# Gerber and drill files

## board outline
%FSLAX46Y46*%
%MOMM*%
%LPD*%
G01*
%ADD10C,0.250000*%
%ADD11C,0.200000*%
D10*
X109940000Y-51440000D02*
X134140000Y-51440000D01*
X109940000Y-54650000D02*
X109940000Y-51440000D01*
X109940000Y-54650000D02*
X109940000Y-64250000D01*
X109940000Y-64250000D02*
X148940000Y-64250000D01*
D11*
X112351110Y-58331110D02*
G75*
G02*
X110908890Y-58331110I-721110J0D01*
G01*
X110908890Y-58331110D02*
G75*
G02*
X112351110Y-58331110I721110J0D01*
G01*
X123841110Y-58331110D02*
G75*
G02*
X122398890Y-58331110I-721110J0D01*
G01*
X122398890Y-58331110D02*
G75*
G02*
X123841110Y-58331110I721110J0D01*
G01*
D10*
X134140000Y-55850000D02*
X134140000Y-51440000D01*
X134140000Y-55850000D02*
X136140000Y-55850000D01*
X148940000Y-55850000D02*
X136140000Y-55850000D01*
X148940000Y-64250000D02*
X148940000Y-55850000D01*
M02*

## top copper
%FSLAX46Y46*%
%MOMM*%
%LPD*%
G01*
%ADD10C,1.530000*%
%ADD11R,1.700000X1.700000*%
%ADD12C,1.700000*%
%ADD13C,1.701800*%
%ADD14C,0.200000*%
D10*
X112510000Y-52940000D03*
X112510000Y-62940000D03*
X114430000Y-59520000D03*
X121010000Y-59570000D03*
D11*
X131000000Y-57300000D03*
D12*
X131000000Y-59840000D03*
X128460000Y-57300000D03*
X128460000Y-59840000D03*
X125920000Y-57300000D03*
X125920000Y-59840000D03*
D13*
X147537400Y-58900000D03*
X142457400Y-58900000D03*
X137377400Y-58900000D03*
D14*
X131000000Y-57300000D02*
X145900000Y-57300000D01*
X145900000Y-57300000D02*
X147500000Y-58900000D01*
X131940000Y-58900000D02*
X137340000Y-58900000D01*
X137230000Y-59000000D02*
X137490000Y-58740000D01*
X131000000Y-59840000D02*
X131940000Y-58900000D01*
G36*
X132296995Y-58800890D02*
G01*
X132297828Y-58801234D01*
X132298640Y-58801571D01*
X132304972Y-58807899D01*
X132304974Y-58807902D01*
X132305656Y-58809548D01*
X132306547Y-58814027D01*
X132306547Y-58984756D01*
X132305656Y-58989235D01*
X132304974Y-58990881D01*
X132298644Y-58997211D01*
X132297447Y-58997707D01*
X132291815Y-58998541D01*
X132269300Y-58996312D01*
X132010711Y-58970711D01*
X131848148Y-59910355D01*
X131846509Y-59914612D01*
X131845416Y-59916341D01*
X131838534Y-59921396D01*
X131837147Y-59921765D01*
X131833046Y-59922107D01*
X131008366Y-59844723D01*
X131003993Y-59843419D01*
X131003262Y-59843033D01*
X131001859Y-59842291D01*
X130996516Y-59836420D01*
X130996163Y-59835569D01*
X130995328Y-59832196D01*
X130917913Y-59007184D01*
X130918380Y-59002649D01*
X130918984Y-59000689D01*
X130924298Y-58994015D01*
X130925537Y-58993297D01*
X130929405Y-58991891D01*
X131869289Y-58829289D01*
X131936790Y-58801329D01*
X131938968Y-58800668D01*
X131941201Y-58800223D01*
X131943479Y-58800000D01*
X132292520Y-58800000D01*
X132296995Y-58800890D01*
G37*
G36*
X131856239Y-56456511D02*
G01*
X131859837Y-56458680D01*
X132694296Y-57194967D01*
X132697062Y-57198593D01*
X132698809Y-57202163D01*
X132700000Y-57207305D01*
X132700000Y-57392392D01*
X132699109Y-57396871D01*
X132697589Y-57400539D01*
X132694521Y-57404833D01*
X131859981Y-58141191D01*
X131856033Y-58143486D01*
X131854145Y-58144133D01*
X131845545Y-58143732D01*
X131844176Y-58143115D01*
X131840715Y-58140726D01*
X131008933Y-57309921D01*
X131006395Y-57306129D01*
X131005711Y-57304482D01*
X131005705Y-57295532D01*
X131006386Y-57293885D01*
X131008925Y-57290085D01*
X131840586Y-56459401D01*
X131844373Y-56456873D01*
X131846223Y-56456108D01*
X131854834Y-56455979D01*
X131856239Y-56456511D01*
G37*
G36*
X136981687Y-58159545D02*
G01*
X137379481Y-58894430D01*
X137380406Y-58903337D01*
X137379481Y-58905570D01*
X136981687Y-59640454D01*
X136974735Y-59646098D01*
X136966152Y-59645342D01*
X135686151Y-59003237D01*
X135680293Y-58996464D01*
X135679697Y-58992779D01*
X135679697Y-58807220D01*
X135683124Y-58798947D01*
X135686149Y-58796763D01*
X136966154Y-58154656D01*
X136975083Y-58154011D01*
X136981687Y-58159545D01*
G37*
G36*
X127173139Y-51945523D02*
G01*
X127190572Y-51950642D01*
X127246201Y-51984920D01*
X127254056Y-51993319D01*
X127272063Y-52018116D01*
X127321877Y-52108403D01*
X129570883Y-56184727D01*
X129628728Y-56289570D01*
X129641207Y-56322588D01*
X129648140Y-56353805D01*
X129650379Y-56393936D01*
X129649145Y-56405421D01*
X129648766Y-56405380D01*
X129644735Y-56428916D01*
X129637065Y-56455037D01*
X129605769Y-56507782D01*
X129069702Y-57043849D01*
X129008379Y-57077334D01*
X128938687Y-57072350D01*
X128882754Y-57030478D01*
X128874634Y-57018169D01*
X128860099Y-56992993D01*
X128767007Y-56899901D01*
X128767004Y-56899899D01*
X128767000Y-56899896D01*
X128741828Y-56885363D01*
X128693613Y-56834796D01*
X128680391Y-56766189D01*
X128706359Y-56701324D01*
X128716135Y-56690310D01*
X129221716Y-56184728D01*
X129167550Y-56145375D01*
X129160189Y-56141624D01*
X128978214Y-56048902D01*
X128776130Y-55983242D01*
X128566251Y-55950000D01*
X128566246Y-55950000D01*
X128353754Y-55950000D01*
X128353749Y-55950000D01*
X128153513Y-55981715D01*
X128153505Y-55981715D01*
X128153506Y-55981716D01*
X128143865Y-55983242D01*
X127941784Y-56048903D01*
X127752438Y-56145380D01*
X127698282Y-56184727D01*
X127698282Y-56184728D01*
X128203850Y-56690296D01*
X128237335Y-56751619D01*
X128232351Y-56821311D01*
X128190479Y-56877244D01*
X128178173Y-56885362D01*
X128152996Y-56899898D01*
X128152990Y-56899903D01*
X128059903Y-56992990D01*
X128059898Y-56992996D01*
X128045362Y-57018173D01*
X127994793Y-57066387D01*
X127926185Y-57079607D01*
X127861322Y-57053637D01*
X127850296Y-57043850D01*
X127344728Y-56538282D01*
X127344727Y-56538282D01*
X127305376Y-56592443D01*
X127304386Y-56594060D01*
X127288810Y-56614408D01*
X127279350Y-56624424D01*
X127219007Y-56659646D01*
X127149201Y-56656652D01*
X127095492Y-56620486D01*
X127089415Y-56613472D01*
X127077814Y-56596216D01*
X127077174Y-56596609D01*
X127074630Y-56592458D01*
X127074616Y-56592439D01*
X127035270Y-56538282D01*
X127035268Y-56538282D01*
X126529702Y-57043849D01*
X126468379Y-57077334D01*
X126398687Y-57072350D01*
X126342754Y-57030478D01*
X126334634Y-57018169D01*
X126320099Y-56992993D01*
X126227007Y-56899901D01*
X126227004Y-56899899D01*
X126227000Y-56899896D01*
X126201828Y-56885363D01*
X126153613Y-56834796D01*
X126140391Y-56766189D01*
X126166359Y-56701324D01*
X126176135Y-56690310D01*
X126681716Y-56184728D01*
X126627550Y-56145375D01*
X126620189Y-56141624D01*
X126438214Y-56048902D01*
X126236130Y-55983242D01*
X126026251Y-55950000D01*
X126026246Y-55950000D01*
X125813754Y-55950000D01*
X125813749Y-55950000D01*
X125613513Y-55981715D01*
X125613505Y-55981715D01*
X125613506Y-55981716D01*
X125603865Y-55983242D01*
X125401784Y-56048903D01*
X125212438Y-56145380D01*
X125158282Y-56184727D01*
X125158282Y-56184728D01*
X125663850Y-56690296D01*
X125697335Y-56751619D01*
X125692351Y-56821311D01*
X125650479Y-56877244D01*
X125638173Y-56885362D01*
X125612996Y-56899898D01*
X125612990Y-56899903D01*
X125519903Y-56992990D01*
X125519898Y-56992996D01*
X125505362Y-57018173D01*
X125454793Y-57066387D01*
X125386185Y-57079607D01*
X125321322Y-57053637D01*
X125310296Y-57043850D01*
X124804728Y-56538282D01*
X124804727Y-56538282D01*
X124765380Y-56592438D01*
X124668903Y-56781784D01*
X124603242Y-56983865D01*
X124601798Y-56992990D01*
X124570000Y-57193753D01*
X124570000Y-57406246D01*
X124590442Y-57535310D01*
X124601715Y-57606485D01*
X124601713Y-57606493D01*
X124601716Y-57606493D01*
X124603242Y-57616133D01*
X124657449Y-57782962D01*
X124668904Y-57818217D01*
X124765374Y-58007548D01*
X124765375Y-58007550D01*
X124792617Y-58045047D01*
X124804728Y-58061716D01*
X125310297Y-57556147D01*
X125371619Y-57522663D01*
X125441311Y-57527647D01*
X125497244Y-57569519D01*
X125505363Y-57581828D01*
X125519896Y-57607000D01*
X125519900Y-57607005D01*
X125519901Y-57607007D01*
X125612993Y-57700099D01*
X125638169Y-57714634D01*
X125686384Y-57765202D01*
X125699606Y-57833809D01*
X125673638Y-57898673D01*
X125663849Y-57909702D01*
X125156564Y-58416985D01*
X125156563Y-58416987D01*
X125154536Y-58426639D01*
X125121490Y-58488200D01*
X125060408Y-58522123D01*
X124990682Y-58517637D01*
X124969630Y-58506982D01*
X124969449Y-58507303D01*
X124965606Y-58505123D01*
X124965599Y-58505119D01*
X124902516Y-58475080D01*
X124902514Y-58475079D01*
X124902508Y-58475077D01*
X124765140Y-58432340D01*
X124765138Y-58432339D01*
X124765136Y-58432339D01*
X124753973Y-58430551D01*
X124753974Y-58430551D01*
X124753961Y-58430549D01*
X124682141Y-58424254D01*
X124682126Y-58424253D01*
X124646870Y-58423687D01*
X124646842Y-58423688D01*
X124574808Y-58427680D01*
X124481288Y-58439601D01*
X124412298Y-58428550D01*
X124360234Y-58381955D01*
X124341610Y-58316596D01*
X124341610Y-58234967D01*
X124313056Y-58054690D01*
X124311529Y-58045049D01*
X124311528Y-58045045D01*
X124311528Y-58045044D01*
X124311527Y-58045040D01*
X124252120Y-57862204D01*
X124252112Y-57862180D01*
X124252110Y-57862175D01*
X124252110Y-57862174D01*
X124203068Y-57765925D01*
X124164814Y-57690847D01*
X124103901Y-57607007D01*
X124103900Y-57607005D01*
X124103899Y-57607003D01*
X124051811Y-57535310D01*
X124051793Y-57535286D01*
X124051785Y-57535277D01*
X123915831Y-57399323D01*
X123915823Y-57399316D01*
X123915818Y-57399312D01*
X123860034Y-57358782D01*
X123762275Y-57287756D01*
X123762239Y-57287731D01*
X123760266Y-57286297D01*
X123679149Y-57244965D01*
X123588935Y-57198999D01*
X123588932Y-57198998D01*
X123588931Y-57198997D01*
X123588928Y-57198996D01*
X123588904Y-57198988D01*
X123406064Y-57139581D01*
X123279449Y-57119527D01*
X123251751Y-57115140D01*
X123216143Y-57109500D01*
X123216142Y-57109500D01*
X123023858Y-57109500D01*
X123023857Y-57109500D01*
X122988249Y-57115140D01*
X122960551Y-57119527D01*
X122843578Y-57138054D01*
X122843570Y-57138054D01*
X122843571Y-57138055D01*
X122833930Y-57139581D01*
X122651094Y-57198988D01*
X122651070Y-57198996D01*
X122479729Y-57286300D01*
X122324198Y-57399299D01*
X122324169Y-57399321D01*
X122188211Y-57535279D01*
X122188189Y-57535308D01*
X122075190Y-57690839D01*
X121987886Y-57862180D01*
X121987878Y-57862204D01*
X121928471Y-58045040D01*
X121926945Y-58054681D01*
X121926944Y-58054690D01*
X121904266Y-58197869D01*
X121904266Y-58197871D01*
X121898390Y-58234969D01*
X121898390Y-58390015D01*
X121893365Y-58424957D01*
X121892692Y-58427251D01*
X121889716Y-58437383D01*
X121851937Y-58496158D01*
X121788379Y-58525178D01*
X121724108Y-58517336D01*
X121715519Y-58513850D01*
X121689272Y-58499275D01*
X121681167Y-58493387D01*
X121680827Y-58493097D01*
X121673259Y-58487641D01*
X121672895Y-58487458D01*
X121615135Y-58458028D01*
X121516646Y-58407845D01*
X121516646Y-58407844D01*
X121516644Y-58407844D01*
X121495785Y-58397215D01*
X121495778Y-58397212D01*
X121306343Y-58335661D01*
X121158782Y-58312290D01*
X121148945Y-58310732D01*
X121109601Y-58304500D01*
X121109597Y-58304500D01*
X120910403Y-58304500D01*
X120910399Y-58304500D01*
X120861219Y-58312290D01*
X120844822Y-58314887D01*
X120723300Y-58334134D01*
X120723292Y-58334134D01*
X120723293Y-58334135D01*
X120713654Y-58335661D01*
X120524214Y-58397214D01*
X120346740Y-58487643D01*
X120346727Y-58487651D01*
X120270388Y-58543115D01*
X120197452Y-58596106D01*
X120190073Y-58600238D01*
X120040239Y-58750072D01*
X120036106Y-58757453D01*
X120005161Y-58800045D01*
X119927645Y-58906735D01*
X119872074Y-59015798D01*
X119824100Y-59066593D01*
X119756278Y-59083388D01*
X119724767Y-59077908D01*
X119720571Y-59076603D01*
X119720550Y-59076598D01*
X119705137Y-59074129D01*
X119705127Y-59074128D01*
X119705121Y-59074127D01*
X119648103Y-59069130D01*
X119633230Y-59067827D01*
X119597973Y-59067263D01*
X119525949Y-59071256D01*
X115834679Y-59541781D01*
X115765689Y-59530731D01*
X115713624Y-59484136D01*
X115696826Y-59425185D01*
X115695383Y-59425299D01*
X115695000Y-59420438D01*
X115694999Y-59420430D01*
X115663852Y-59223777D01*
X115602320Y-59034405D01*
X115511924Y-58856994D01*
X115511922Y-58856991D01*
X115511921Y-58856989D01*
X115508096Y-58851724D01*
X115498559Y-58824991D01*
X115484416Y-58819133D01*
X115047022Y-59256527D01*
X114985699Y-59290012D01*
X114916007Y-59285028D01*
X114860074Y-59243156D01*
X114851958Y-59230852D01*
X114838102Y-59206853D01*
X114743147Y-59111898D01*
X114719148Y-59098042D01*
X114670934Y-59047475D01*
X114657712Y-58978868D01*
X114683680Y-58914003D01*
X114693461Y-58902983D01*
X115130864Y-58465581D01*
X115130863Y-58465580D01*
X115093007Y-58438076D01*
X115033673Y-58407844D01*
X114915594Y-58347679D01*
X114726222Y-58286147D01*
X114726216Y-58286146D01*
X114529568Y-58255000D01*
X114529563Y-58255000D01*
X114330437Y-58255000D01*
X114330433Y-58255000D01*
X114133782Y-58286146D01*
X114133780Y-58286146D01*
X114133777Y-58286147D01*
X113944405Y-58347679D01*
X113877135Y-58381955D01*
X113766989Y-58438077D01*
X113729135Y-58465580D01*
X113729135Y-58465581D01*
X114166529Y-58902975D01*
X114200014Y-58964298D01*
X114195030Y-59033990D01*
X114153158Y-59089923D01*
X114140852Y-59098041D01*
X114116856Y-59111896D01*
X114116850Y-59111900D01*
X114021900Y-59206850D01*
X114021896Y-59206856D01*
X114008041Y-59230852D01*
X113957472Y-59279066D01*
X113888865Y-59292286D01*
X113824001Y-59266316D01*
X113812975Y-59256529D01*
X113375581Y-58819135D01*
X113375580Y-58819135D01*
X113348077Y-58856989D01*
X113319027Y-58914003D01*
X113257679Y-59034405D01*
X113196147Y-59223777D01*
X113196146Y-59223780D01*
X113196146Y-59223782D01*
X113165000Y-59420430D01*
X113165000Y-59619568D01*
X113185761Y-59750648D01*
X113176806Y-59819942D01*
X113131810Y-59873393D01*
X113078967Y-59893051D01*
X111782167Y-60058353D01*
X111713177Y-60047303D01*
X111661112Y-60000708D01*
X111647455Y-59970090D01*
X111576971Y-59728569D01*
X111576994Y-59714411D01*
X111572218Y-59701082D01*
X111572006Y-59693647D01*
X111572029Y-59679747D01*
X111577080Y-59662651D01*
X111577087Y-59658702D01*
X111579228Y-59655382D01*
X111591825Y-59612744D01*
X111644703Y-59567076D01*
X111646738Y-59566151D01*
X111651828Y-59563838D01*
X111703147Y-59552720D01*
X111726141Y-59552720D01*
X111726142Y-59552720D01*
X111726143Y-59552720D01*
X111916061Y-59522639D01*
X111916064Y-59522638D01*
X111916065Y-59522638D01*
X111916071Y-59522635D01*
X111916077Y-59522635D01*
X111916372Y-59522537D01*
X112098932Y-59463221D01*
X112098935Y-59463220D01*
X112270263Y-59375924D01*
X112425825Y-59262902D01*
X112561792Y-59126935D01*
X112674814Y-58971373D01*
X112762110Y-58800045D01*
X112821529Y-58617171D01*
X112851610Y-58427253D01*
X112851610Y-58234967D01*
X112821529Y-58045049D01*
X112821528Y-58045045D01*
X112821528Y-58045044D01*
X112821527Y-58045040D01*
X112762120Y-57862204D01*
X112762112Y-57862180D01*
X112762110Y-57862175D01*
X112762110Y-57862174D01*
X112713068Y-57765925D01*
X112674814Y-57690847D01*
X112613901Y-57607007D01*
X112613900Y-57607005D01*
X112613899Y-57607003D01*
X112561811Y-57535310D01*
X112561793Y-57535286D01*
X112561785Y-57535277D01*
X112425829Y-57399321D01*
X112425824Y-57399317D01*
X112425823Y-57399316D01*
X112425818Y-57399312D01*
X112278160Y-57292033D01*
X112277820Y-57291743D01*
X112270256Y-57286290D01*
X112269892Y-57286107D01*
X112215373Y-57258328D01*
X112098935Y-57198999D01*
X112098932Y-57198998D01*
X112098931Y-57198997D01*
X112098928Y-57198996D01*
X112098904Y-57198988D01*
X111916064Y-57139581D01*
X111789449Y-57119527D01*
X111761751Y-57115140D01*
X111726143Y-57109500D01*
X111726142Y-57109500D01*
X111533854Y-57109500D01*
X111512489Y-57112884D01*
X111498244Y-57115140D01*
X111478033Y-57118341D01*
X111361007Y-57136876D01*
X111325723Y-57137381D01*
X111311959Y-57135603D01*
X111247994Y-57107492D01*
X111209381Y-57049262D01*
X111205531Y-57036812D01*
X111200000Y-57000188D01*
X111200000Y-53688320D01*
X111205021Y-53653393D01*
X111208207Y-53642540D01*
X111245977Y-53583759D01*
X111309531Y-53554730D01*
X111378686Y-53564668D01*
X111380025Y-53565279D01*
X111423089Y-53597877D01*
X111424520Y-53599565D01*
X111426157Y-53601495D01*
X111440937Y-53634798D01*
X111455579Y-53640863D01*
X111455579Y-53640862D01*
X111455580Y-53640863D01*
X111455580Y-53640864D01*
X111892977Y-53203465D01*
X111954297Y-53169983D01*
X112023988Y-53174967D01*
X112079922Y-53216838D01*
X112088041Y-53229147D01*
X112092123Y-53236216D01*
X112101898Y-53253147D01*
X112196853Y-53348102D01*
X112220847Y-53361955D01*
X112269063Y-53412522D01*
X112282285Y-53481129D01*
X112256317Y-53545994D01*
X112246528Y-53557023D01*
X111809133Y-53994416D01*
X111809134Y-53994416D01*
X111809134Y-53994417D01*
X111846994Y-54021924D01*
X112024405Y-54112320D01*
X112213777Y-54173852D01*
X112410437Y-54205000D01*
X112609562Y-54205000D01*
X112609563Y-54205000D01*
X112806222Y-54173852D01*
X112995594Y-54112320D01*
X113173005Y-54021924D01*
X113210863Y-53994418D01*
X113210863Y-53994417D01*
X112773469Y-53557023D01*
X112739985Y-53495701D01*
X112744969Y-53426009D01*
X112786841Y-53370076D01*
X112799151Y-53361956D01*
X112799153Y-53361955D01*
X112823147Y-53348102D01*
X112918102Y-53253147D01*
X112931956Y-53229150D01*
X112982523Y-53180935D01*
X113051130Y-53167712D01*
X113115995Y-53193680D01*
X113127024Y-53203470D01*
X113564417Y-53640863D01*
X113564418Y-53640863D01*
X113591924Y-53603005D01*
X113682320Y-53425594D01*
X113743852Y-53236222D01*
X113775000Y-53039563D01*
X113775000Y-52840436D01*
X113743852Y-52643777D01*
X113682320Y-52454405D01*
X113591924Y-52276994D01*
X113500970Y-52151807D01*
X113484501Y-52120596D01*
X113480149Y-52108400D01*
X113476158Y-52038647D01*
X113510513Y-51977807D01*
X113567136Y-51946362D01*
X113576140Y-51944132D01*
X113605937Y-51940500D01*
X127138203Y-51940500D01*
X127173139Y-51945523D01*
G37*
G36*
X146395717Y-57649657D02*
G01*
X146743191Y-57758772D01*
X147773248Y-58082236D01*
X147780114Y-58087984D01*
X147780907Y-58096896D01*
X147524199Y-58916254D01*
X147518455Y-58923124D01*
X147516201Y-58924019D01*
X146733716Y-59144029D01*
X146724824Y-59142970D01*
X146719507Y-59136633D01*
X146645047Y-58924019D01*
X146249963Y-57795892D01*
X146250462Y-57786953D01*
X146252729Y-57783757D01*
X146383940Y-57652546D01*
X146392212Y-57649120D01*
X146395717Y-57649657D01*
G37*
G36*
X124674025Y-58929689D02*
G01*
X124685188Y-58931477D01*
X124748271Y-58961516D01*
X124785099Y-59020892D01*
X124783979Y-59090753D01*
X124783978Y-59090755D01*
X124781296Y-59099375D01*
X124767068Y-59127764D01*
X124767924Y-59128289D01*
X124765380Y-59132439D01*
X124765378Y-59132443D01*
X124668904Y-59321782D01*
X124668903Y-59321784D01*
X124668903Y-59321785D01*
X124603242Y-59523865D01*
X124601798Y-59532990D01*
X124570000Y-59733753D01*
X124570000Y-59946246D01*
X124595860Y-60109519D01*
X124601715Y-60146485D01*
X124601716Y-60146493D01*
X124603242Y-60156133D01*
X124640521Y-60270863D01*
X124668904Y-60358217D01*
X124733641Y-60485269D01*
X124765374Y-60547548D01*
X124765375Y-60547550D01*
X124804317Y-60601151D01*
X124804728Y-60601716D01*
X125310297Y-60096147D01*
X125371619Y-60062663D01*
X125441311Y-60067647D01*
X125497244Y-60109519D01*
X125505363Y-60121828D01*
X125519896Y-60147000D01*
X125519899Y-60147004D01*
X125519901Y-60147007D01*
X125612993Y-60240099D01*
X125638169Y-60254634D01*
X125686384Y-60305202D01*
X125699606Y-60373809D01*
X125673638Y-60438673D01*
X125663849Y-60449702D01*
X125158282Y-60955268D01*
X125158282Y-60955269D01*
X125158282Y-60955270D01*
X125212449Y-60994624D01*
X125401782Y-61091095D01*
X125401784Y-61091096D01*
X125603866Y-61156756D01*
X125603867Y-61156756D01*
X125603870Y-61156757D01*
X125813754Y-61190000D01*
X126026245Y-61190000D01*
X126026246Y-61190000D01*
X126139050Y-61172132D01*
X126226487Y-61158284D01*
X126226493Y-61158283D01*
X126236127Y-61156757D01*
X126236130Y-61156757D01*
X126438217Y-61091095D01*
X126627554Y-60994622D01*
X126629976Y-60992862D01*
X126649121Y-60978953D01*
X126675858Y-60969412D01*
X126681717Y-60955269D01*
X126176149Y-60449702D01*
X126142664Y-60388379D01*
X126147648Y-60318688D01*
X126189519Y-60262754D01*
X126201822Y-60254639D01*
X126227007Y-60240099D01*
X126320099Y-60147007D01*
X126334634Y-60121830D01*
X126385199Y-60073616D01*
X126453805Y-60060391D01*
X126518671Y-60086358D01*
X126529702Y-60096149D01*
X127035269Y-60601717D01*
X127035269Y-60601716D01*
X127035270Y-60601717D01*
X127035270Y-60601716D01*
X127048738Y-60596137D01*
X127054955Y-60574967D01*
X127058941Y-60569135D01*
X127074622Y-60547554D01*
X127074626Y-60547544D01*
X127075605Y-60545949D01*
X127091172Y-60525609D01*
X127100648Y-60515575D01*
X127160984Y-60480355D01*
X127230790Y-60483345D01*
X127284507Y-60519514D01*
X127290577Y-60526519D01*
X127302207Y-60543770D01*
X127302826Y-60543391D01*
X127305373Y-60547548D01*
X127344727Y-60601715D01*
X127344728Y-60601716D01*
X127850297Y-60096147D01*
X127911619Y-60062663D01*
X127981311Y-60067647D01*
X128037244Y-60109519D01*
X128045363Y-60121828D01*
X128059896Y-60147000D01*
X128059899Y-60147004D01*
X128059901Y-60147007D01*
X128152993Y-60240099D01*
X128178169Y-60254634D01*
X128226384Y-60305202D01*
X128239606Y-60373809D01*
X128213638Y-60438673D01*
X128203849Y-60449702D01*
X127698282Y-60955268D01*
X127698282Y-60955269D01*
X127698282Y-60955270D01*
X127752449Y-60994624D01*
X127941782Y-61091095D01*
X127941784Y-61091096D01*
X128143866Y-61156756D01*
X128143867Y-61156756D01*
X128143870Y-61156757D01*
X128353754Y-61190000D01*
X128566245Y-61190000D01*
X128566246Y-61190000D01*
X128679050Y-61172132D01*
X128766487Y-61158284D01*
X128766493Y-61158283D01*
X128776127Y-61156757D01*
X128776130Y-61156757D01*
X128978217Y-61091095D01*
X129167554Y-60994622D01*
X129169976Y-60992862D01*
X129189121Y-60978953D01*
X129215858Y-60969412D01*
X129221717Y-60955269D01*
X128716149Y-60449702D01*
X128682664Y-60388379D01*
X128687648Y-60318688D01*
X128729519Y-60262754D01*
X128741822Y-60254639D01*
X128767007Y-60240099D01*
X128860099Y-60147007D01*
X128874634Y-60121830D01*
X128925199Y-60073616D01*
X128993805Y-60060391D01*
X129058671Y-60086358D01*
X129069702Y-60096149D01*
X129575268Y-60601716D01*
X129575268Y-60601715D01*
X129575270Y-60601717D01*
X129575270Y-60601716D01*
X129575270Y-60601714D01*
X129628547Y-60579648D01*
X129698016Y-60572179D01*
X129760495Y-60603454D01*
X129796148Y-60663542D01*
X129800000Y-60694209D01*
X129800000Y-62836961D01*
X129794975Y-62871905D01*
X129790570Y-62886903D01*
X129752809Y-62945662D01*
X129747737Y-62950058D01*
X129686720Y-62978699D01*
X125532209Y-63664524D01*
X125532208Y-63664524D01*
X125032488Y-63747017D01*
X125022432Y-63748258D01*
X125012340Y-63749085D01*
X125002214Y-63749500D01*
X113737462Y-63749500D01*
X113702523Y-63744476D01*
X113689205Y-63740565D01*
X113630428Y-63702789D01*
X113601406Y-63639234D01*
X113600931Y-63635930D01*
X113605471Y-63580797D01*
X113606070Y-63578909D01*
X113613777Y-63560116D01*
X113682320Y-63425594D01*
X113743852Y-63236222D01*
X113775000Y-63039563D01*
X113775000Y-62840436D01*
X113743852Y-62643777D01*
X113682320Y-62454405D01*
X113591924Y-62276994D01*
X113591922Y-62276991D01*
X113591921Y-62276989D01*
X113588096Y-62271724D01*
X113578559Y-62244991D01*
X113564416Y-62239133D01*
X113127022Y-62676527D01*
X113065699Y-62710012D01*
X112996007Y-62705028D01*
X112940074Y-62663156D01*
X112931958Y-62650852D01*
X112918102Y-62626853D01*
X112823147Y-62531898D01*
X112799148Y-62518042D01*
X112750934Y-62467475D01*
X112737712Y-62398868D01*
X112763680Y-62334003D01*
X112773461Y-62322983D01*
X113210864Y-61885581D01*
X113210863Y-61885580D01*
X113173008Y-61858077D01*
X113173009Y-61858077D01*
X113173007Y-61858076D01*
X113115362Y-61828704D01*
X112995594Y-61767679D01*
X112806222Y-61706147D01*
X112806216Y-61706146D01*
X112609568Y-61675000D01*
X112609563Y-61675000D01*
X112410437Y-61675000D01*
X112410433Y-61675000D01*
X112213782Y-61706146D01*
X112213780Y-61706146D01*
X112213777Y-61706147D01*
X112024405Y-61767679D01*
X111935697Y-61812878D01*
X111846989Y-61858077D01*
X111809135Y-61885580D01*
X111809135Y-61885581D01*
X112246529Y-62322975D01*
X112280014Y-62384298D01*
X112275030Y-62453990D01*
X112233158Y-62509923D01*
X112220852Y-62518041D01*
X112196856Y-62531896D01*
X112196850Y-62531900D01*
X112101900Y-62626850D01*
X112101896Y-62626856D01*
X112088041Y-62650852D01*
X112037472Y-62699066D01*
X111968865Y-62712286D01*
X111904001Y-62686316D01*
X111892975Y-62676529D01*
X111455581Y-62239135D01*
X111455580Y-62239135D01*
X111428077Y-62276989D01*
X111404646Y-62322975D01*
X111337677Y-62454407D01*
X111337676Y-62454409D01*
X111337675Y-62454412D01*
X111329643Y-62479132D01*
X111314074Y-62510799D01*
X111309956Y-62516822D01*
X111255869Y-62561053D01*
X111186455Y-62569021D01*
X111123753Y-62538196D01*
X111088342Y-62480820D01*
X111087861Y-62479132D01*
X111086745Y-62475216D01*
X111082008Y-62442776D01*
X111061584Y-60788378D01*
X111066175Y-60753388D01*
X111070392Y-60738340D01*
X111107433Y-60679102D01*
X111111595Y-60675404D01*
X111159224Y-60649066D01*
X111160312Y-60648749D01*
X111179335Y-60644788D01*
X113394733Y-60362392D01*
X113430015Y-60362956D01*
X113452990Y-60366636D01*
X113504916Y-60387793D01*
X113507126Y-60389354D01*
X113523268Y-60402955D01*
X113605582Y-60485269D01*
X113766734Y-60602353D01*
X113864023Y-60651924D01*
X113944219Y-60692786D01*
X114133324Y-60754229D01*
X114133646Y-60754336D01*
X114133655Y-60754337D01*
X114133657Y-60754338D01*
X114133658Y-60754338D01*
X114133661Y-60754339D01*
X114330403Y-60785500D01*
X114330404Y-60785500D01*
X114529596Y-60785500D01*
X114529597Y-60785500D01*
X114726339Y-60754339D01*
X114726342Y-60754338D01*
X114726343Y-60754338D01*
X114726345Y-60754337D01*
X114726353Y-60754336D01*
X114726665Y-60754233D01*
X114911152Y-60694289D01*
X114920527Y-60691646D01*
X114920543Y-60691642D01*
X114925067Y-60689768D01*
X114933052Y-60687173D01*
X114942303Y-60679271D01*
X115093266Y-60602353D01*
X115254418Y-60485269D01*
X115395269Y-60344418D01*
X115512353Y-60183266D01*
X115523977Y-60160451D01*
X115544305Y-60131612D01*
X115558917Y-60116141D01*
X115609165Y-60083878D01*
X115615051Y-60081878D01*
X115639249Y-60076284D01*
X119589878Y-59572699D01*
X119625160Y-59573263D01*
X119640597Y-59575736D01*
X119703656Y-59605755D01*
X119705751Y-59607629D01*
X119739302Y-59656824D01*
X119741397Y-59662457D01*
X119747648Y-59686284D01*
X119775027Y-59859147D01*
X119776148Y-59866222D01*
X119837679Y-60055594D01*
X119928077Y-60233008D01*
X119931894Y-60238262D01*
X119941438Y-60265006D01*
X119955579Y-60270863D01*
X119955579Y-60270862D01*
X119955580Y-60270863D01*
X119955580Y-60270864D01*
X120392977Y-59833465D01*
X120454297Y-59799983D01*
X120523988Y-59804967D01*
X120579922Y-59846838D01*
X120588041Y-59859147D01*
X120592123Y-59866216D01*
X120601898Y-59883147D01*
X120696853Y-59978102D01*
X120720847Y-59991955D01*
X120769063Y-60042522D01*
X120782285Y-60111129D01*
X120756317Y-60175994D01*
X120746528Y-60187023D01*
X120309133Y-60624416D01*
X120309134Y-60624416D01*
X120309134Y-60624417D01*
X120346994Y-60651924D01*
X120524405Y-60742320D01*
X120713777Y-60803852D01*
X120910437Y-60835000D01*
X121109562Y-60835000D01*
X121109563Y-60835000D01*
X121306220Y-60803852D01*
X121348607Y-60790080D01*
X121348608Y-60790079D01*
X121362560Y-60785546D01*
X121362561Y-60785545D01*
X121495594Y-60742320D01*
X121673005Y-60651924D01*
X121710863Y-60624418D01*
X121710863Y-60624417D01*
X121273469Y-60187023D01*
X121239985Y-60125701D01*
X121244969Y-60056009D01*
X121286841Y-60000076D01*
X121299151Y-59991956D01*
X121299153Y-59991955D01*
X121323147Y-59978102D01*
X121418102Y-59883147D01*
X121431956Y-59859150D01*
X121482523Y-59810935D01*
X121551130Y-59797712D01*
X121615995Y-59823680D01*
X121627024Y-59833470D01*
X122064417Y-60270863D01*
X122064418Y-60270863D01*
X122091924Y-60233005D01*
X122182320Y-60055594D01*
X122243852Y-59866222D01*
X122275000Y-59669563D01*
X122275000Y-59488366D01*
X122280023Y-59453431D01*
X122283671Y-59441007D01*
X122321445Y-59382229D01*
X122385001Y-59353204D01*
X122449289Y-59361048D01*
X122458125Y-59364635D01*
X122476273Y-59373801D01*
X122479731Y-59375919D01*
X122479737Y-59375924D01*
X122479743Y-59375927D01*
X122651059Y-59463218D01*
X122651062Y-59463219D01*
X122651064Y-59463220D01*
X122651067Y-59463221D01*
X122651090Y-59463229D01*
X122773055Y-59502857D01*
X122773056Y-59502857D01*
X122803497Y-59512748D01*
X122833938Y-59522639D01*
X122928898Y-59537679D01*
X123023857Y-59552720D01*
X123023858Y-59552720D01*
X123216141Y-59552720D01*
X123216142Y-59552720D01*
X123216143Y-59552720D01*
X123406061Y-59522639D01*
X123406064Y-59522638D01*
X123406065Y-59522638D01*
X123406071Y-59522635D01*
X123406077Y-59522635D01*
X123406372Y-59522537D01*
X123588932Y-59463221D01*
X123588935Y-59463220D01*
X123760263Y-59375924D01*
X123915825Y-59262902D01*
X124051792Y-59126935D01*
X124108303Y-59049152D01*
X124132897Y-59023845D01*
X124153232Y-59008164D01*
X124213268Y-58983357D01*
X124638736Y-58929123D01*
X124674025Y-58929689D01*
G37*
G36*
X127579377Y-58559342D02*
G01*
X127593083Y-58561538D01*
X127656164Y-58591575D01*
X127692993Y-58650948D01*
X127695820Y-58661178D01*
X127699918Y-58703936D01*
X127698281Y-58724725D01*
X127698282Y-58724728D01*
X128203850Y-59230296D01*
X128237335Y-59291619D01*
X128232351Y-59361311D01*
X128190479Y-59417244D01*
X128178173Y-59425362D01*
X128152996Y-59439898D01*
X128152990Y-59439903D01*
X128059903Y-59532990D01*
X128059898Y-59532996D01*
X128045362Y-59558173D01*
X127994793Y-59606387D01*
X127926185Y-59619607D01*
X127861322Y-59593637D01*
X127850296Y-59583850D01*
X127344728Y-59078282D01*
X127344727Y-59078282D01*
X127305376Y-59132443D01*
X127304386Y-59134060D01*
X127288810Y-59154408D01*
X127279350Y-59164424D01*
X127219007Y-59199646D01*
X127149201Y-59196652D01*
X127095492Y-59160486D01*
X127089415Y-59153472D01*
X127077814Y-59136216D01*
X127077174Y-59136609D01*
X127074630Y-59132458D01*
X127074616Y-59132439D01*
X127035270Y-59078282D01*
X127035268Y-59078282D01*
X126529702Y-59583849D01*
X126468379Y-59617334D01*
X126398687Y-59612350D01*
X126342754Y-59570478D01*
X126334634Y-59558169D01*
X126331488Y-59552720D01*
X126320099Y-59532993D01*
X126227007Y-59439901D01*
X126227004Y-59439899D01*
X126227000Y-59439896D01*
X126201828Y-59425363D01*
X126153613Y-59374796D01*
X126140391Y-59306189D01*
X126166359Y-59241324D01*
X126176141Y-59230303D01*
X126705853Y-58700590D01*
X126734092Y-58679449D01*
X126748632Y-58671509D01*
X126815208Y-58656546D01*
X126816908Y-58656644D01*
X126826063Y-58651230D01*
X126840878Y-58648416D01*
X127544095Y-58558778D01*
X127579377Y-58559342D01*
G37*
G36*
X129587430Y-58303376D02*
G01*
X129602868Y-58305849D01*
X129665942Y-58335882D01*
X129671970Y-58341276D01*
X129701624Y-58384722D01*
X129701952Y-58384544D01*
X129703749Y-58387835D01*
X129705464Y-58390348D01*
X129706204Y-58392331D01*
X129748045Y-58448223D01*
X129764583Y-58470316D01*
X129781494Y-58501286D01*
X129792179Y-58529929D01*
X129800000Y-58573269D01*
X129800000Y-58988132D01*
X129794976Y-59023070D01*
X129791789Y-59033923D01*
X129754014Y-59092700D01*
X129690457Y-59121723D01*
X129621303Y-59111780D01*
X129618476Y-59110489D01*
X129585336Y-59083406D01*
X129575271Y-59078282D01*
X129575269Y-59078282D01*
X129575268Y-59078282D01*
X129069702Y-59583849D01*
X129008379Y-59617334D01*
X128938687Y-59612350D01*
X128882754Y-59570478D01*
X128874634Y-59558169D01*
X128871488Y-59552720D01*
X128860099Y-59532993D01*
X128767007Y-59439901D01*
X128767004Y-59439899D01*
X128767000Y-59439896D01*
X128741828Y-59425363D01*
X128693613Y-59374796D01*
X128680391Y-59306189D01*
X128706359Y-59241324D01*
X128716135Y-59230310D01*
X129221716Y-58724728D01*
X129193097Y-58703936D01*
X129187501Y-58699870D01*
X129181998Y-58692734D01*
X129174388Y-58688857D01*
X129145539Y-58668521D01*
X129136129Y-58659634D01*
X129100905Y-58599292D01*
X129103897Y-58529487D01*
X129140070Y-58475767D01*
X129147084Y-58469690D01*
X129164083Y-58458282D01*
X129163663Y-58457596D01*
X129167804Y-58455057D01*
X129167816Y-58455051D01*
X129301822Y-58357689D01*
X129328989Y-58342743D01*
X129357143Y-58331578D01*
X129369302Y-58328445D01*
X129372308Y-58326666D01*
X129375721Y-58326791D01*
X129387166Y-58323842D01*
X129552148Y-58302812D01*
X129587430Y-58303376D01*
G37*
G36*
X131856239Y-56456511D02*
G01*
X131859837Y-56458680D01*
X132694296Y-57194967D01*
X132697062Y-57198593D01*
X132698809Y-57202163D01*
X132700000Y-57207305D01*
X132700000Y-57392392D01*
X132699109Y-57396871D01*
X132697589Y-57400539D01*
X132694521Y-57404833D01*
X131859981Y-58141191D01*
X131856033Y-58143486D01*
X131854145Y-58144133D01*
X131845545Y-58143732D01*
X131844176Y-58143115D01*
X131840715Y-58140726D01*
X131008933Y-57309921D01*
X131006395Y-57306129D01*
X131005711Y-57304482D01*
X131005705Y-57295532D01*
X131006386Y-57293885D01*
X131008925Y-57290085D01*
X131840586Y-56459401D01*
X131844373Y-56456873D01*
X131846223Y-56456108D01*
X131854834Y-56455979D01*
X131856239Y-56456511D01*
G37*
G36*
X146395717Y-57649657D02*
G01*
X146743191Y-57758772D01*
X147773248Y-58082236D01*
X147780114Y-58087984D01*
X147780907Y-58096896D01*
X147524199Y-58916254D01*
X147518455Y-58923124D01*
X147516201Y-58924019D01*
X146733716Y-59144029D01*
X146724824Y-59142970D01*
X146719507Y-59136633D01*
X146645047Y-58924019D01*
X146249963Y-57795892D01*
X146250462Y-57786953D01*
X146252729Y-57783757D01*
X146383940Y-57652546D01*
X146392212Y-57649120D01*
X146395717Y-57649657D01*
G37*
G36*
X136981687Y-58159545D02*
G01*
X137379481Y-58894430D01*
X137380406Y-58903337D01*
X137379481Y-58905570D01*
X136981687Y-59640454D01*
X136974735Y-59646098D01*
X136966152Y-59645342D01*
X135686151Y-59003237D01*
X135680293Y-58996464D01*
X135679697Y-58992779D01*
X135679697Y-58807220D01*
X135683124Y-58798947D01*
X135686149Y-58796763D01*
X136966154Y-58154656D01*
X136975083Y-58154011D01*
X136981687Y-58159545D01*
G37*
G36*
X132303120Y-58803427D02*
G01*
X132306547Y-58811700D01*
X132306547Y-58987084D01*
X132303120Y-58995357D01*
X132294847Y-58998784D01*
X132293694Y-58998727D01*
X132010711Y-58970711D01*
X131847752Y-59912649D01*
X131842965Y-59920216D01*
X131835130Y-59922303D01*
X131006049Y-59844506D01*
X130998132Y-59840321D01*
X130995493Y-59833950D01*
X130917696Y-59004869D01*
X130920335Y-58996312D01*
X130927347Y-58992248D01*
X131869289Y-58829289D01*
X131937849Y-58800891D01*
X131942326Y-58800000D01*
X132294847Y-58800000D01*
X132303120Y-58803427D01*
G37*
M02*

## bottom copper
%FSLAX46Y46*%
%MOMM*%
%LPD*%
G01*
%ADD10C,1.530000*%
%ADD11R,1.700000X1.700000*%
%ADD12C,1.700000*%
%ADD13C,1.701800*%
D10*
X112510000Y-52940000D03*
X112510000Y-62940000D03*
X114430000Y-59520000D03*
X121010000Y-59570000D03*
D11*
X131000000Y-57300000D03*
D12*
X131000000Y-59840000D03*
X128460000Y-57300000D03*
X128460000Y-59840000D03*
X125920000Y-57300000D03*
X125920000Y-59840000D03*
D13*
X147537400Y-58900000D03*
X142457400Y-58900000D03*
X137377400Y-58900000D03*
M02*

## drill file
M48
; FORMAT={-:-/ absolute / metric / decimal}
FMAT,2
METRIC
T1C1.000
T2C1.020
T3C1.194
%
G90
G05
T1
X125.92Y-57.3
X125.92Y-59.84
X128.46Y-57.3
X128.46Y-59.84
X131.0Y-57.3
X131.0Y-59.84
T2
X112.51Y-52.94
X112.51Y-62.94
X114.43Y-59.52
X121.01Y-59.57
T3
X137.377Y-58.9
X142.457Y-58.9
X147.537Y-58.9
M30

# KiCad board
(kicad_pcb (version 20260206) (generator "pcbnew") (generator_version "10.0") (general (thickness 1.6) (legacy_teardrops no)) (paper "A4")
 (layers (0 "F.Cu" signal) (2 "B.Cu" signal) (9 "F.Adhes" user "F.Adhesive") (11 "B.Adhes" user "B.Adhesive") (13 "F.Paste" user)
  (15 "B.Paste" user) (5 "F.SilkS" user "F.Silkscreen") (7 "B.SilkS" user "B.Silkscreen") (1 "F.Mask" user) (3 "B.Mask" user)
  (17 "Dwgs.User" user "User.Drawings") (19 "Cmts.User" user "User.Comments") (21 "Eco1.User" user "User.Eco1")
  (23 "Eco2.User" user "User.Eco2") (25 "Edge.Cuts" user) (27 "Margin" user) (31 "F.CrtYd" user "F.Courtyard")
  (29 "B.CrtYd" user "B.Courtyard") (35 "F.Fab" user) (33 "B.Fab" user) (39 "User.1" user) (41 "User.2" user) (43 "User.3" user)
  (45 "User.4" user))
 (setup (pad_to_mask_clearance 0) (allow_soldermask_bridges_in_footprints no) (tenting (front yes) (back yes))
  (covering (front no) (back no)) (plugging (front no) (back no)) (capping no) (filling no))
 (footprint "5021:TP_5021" (layer "F.Cu") (at 112.51 52.94 -90)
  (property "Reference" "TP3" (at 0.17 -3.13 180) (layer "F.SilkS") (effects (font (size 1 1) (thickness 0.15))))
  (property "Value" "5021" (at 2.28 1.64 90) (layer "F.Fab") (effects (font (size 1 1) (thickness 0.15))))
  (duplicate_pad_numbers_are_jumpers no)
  (pad "TP" thru_hole circle (at 0 0 270) (size 1.53 1.53) (drill 1.02) (layers "*.Cu" "*.Mask") (remove_unused_layers no)
   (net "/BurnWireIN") (solder_mask_margin 0.102)
   (teardrops (best_length_ratio 0.5) (max_length 1) (best_width_ratio 1) (max_width 2) (curved_edges no) (filter_ratio 0.9) (enabled yes)
    (allow_two_segments yes) (prefer_zone_connections yes))))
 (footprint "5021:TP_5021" (layer "F.Cu") (at 112.51 62.94 -90)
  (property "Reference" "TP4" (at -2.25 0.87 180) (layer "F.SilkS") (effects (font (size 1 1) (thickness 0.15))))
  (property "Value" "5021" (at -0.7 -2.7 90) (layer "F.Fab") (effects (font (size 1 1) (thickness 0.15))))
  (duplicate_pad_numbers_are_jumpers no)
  (pad "TP" thru_hole circle (at 0 0 270) (size 1.53 1.53) (drill 1.02) (layers "*.Cu" "*.Mask") (remove_unused_layers no) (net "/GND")
   (solder_mask_margin 0.102)
   (teardrops (best_length_ratio 0.5) (max_length 1) (best_width_ratio 1) (max_width 2) (curved_edges no) (filter_ratio 0.9) (enabled yes)
    (allow_two_segments yes) (prefer_zone_connections yes))))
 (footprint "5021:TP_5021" (layer "F.Cu") (at 114.43 59.52)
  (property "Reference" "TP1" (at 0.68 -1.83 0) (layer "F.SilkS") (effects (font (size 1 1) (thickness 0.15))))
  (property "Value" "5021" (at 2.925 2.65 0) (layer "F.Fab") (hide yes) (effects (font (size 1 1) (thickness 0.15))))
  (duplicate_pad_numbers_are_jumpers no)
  (pad "TP" thru_hole circle (at 0 0) (size 1.53 1.53) (drill 1.02) (layers "*.Cu" "*.Mask") (remove_unused_layers no) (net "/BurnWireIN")
   (solder_mask_margin 0.102)
   (teardrops (best_length_ratio 0.5) (max_length 1) (best_width_ratio 1) (max_width 2) (curved_edges no) (filter_ratio 0.9) (enabled yes)
    (allow_two_segments yes) (prefer_zone_connections yes))))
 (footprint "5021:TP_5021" (layer "F.Cu") (at 121.01 59.57)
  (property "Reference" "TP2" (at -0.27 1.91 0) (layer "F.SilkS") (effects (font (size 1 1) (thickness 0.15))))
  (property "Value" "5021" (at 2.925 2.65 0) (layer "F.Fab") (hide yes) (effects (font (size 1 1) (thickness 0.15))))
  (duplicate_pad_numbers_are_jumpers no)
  (pad "TP" thru_hole circle (at 0 0) (size 1.53 1.53) (drill 1.02) (layers "*.Cu" "*.Mask") (remove_unused_layers no) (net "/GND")
   (solder_mask_margin 0.102)
   (teardrops (best_length_ratio 0.5) (max_length 1) (best_width_ratio 1) (max_width 2) (curved_edges no) (filter_ratio 0.9) (enabled yes)
    (allow_two_segments yes) (prefer_zone_connections yes))))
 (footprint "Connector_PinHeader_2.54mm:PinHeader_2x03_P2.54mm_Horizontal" (layer "F.Cu") (at 131 57.3 -90)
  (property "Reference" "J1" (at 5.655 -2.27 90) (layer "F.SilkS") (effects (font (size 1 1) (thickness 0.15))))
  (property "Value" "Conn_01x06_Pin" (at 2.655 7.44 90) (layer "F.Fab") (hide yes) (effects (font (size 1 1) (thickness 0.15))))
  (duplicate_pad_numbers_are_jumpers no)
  (pad "1" thru_hole rect (at 0 0 270) (size 1.7 1.7) (drill 1) (layers "*.Cu" "*.Mask") (remove_unused_layers no)
   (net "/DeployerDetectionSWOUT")
   (teardrops (best_length_ratio 0.5) (max_length 1) (best_width_ratio 1) (max_width 2) (curved_edges no) (filter_ratio 0.9) (enabled yes)
    (allow_two_segments yes) (prefer_zone_connections yes)))
  (pad "2" thru_hole circle (at 2.54 0 270) (size 1.7 1.7) (drill 1) (layers "*.Cu" "*.Mask") (remove_unused_layers no)
   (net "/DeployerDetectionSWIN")
   (teardrops (best_length_ratio 0.5) (max_length 1) (best_width_ratio 1) (max_width 2) (curved_edges no) (filter_ratio 0.9) (enabled yes)
    (allow_two_segments yes) (prefer_zone_connections yes)))
  (pad "3" thru_hole circle (at 0 2.54 270) (size 1.7 1.7) (drill 1) (layers "*.Cu" "*.Mask") (remove_unused_layers no) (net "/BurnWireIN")
   (teardrops (best_length_ratio 0.5) (max_length 1) (best_width_ratio 1) (max_width 2) (curved_edges no) (filter_ratio 0.9) (enabled yes)
    (allow_two_segments yes) (prefer_zone_connections yes)))
  (pad "4" thru_hole circle (at 2.54 2.54 270) (size 1.7 1.7) (drill 1) (layers "*.Cu" "*.Mask") (remove_unused_layers no) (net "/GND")
   (teardrops (best_length_ratio 0.5) (max_length 1) (best_width_ratio 1) (max_width 2) (curved_edges no) (filter_ratio 0.9) (enabled yes)
    (allow_two_segments yes) (prefer_zone_connections yes)))
  (pad "5" thru_hole circle (at 0 5.08 270) (size 1.7 1.7) (drill 1) (layers "*.Cu" "*.Mask") (remove_unused_layers no) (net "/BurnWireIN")
   (teardrops (best_length_ratio 0.5) (max_length 1) (best_width_ratio 1) (max_width 2) (curved_edges no) (filter_ratio 0.9) (enabled yes)
    (allow_two_segments yes) (prefer_zone_connections yes)))
  (pad "6" thru_hole circle (at 2.54 5.08 270) (size 1.7 1.7) (drill 1) (layers "*.Cu" "*.Mask") (remove_unused_layers no) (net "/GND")
   (teardrops (best_length_ratio 0.5) (max_length 1) (best_width_ratio 1) (max_width 2) (curved_edges no) (filter_ratio 0.9) (enabled yes)
    (allow_two_segments yes) (prefer_zone_connections yes))))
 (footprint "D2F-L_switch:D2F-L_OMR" (layer "B.Cu") (at 147.5374 58.9 180)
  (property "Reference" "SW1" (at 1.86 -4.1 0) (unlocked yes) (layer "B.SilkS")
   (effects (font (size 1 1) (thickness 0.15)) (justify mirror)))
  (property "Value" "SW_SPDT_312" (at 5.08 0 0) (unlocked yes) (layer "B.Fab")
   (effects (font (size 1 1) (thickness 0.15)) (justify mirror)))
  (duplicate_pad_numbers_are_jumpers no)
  (pad "1" thru_hole circle (at 0 0 180) (size 1.7018 1.7018) (drill 1.1938) (layers "*.Cu" "*.Mask") (remove_unused_layers no)
   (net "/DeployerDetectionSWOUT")
   (teardrops (best_length_ratio 0.5) (max_length 1) (best_width_ratio 1) (max_width 2) (curved_edges no) (filter_ratio 0.9) (enabled yes)
    (allow_two_segments yes) (prefer_zone_connections yes)))
  (pad "2" thru_hole circle (at 5.08 0 180) (size 1.7018 1.7018) (drill 1.1938) (layers "*.Cu" "*.Mask") (remove_unused_layers no)
   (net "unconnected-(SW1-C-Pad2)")
   (teardrops (best_length_ratio 0.5) (max_length 1) (best_width_ratio 1) (max_width 2) (curved_edges no) (filter_ratio 0.9) (enabled yes)
    (allow_two_segments yes) (prefer_zone_connections yes)))
  (pad "3" thru_hole circle (at 10.16 0 180) (size 1.7018 1.7018) (drill 1.1938) (layers "*.Cu" "*.Mask") (remove_unused_layers no)
   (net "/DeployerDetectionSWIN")
   (teardrops (best_length_ratio 0.5) (max_length 1) (best_width_ratio 1) (max_width 2) (curved_edges no) (filter_ratio 0.9) (enabled yes)
    (allow_two_segments yes) (prefer_zone_connections yes))))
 (gr_line (start 109.94 51.44) (end 134.14 51.44) (stroke (width 0.25) (type solid)) (layer "Edge.Cuts"))
 (gr_line (start 109.94 54.65) (end 109.94 51.44) (stroke (width 0.25) (type solid)) (layer "Edge.Cuts"))
 (gr_line (start 109.94 54.65) (end 109.94 64.25) (stroke (width 0.25) (type default)) (layer "Edge.Cuts"))
 (gr_line (start 109.94 64.25) (end 148.94 64.25) (stroke (width 0.25) (type solid)) (layer "Edge.Cuts"))
 (gr_circle (center 111.63 58.33111) (end 112.23 58.73111) (stroke (width 0.2) (type solid)) (fill no) (layer "Edge.Cuts"))
 (gr_circle (center 123.12 58.33111) (end 123.84111 58.33111) (stroke (width 0.2) (type solid)) (fill no) (layer "Edge.Cuts"))
 (gr_line (start 134.14 55.85) (end 134.14 51.44) (stroke (width 0.25) (type solid)) (layer "Edge.Cuts"))
 (gr_line (start 134.14 55.85) (end 136.14 55.85) (stroke (width 0.25) (type solid)) (layer "Edge.Cuts"))
 (gr_line (start 148.94 55.85) (end 136.14 55.85) (stroke (width 0.25) (type default)) (layer "Edge.Cuts"))
 (gr_line (start 148.94 64.25) (end 148.94 55.85) (stroke (width 0.25) (type default)) (layer "Edge.Cuts"))
 (segment (start 131 57.3) (end 145.9 57.3) (width 0.2) (layer "F.Cu") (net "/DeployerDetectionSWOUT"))
 (segment (start 145.9 57.3) (end 147.5 58.9) (width 0.2) (layer "F.Cu") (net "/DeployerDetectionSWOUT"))
 (segment (start 131.94 58.9) (end 137.34 58.9) (width 0.2) (layer "F.Cu") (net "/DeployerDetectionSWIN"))
 (segment (start 137.23 59) (end 137.49 58.74) (width 0.2) (layer "F.Cu") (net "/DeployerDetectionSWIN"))
 (segment (start 131 59.84) (end 131.94 58.9) (width 0.2) (layer "F.Cu") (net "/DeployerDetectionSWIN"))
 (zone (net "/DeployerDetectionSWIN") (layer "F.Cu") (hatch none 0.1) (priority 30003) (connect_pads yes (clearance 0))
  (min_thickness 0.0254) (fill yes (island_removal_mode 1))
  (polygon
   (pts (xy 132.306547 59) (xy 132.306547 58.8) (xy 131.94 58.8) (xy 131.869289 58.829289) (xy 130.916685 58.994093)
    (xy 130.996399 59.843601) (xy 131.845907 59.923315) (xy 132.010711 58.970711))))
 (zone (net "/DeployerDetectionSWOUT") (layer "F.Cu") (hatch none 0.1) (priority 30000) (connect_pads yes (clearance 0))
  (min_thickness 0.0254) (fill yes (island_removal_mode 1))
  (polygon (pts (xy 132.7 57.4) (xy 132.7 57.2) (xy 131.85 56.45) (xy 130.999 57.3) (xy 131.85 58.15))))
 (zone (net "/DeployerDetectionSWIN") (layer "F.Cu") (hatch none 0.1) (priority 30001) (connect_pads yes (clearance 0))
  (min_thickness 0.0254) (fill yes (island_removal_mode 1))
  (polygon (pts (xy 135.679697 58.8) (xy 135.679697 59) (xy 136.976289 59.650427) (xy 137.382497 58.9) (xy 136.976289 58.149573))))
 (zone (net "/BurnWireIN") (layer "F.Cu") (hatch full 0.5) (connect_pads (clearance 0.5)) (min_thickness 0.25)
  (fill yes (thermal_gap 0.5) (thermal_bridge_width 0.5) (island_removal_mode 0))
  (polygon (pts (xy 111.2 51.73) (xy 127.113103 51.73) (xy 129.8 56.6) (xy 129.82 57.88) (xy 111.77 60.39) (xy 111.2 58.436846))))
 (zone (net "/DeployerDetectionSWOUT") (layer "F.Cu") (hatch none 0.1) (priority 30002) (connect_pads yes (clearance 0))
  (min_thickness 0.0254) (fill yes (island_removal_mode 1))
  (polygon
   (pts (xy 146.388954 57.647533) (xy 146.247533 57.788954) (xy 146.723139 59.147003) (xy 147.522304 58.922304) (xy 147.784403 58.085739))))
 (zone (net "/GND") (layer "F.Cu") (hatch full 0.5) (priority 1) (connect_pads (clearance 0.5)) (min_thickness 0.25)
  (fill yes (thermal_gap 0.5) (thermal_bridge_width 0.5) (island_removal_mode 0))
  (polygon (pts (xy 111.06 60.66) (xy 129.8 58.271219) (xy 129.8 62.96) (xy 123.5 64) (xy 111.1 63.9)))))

